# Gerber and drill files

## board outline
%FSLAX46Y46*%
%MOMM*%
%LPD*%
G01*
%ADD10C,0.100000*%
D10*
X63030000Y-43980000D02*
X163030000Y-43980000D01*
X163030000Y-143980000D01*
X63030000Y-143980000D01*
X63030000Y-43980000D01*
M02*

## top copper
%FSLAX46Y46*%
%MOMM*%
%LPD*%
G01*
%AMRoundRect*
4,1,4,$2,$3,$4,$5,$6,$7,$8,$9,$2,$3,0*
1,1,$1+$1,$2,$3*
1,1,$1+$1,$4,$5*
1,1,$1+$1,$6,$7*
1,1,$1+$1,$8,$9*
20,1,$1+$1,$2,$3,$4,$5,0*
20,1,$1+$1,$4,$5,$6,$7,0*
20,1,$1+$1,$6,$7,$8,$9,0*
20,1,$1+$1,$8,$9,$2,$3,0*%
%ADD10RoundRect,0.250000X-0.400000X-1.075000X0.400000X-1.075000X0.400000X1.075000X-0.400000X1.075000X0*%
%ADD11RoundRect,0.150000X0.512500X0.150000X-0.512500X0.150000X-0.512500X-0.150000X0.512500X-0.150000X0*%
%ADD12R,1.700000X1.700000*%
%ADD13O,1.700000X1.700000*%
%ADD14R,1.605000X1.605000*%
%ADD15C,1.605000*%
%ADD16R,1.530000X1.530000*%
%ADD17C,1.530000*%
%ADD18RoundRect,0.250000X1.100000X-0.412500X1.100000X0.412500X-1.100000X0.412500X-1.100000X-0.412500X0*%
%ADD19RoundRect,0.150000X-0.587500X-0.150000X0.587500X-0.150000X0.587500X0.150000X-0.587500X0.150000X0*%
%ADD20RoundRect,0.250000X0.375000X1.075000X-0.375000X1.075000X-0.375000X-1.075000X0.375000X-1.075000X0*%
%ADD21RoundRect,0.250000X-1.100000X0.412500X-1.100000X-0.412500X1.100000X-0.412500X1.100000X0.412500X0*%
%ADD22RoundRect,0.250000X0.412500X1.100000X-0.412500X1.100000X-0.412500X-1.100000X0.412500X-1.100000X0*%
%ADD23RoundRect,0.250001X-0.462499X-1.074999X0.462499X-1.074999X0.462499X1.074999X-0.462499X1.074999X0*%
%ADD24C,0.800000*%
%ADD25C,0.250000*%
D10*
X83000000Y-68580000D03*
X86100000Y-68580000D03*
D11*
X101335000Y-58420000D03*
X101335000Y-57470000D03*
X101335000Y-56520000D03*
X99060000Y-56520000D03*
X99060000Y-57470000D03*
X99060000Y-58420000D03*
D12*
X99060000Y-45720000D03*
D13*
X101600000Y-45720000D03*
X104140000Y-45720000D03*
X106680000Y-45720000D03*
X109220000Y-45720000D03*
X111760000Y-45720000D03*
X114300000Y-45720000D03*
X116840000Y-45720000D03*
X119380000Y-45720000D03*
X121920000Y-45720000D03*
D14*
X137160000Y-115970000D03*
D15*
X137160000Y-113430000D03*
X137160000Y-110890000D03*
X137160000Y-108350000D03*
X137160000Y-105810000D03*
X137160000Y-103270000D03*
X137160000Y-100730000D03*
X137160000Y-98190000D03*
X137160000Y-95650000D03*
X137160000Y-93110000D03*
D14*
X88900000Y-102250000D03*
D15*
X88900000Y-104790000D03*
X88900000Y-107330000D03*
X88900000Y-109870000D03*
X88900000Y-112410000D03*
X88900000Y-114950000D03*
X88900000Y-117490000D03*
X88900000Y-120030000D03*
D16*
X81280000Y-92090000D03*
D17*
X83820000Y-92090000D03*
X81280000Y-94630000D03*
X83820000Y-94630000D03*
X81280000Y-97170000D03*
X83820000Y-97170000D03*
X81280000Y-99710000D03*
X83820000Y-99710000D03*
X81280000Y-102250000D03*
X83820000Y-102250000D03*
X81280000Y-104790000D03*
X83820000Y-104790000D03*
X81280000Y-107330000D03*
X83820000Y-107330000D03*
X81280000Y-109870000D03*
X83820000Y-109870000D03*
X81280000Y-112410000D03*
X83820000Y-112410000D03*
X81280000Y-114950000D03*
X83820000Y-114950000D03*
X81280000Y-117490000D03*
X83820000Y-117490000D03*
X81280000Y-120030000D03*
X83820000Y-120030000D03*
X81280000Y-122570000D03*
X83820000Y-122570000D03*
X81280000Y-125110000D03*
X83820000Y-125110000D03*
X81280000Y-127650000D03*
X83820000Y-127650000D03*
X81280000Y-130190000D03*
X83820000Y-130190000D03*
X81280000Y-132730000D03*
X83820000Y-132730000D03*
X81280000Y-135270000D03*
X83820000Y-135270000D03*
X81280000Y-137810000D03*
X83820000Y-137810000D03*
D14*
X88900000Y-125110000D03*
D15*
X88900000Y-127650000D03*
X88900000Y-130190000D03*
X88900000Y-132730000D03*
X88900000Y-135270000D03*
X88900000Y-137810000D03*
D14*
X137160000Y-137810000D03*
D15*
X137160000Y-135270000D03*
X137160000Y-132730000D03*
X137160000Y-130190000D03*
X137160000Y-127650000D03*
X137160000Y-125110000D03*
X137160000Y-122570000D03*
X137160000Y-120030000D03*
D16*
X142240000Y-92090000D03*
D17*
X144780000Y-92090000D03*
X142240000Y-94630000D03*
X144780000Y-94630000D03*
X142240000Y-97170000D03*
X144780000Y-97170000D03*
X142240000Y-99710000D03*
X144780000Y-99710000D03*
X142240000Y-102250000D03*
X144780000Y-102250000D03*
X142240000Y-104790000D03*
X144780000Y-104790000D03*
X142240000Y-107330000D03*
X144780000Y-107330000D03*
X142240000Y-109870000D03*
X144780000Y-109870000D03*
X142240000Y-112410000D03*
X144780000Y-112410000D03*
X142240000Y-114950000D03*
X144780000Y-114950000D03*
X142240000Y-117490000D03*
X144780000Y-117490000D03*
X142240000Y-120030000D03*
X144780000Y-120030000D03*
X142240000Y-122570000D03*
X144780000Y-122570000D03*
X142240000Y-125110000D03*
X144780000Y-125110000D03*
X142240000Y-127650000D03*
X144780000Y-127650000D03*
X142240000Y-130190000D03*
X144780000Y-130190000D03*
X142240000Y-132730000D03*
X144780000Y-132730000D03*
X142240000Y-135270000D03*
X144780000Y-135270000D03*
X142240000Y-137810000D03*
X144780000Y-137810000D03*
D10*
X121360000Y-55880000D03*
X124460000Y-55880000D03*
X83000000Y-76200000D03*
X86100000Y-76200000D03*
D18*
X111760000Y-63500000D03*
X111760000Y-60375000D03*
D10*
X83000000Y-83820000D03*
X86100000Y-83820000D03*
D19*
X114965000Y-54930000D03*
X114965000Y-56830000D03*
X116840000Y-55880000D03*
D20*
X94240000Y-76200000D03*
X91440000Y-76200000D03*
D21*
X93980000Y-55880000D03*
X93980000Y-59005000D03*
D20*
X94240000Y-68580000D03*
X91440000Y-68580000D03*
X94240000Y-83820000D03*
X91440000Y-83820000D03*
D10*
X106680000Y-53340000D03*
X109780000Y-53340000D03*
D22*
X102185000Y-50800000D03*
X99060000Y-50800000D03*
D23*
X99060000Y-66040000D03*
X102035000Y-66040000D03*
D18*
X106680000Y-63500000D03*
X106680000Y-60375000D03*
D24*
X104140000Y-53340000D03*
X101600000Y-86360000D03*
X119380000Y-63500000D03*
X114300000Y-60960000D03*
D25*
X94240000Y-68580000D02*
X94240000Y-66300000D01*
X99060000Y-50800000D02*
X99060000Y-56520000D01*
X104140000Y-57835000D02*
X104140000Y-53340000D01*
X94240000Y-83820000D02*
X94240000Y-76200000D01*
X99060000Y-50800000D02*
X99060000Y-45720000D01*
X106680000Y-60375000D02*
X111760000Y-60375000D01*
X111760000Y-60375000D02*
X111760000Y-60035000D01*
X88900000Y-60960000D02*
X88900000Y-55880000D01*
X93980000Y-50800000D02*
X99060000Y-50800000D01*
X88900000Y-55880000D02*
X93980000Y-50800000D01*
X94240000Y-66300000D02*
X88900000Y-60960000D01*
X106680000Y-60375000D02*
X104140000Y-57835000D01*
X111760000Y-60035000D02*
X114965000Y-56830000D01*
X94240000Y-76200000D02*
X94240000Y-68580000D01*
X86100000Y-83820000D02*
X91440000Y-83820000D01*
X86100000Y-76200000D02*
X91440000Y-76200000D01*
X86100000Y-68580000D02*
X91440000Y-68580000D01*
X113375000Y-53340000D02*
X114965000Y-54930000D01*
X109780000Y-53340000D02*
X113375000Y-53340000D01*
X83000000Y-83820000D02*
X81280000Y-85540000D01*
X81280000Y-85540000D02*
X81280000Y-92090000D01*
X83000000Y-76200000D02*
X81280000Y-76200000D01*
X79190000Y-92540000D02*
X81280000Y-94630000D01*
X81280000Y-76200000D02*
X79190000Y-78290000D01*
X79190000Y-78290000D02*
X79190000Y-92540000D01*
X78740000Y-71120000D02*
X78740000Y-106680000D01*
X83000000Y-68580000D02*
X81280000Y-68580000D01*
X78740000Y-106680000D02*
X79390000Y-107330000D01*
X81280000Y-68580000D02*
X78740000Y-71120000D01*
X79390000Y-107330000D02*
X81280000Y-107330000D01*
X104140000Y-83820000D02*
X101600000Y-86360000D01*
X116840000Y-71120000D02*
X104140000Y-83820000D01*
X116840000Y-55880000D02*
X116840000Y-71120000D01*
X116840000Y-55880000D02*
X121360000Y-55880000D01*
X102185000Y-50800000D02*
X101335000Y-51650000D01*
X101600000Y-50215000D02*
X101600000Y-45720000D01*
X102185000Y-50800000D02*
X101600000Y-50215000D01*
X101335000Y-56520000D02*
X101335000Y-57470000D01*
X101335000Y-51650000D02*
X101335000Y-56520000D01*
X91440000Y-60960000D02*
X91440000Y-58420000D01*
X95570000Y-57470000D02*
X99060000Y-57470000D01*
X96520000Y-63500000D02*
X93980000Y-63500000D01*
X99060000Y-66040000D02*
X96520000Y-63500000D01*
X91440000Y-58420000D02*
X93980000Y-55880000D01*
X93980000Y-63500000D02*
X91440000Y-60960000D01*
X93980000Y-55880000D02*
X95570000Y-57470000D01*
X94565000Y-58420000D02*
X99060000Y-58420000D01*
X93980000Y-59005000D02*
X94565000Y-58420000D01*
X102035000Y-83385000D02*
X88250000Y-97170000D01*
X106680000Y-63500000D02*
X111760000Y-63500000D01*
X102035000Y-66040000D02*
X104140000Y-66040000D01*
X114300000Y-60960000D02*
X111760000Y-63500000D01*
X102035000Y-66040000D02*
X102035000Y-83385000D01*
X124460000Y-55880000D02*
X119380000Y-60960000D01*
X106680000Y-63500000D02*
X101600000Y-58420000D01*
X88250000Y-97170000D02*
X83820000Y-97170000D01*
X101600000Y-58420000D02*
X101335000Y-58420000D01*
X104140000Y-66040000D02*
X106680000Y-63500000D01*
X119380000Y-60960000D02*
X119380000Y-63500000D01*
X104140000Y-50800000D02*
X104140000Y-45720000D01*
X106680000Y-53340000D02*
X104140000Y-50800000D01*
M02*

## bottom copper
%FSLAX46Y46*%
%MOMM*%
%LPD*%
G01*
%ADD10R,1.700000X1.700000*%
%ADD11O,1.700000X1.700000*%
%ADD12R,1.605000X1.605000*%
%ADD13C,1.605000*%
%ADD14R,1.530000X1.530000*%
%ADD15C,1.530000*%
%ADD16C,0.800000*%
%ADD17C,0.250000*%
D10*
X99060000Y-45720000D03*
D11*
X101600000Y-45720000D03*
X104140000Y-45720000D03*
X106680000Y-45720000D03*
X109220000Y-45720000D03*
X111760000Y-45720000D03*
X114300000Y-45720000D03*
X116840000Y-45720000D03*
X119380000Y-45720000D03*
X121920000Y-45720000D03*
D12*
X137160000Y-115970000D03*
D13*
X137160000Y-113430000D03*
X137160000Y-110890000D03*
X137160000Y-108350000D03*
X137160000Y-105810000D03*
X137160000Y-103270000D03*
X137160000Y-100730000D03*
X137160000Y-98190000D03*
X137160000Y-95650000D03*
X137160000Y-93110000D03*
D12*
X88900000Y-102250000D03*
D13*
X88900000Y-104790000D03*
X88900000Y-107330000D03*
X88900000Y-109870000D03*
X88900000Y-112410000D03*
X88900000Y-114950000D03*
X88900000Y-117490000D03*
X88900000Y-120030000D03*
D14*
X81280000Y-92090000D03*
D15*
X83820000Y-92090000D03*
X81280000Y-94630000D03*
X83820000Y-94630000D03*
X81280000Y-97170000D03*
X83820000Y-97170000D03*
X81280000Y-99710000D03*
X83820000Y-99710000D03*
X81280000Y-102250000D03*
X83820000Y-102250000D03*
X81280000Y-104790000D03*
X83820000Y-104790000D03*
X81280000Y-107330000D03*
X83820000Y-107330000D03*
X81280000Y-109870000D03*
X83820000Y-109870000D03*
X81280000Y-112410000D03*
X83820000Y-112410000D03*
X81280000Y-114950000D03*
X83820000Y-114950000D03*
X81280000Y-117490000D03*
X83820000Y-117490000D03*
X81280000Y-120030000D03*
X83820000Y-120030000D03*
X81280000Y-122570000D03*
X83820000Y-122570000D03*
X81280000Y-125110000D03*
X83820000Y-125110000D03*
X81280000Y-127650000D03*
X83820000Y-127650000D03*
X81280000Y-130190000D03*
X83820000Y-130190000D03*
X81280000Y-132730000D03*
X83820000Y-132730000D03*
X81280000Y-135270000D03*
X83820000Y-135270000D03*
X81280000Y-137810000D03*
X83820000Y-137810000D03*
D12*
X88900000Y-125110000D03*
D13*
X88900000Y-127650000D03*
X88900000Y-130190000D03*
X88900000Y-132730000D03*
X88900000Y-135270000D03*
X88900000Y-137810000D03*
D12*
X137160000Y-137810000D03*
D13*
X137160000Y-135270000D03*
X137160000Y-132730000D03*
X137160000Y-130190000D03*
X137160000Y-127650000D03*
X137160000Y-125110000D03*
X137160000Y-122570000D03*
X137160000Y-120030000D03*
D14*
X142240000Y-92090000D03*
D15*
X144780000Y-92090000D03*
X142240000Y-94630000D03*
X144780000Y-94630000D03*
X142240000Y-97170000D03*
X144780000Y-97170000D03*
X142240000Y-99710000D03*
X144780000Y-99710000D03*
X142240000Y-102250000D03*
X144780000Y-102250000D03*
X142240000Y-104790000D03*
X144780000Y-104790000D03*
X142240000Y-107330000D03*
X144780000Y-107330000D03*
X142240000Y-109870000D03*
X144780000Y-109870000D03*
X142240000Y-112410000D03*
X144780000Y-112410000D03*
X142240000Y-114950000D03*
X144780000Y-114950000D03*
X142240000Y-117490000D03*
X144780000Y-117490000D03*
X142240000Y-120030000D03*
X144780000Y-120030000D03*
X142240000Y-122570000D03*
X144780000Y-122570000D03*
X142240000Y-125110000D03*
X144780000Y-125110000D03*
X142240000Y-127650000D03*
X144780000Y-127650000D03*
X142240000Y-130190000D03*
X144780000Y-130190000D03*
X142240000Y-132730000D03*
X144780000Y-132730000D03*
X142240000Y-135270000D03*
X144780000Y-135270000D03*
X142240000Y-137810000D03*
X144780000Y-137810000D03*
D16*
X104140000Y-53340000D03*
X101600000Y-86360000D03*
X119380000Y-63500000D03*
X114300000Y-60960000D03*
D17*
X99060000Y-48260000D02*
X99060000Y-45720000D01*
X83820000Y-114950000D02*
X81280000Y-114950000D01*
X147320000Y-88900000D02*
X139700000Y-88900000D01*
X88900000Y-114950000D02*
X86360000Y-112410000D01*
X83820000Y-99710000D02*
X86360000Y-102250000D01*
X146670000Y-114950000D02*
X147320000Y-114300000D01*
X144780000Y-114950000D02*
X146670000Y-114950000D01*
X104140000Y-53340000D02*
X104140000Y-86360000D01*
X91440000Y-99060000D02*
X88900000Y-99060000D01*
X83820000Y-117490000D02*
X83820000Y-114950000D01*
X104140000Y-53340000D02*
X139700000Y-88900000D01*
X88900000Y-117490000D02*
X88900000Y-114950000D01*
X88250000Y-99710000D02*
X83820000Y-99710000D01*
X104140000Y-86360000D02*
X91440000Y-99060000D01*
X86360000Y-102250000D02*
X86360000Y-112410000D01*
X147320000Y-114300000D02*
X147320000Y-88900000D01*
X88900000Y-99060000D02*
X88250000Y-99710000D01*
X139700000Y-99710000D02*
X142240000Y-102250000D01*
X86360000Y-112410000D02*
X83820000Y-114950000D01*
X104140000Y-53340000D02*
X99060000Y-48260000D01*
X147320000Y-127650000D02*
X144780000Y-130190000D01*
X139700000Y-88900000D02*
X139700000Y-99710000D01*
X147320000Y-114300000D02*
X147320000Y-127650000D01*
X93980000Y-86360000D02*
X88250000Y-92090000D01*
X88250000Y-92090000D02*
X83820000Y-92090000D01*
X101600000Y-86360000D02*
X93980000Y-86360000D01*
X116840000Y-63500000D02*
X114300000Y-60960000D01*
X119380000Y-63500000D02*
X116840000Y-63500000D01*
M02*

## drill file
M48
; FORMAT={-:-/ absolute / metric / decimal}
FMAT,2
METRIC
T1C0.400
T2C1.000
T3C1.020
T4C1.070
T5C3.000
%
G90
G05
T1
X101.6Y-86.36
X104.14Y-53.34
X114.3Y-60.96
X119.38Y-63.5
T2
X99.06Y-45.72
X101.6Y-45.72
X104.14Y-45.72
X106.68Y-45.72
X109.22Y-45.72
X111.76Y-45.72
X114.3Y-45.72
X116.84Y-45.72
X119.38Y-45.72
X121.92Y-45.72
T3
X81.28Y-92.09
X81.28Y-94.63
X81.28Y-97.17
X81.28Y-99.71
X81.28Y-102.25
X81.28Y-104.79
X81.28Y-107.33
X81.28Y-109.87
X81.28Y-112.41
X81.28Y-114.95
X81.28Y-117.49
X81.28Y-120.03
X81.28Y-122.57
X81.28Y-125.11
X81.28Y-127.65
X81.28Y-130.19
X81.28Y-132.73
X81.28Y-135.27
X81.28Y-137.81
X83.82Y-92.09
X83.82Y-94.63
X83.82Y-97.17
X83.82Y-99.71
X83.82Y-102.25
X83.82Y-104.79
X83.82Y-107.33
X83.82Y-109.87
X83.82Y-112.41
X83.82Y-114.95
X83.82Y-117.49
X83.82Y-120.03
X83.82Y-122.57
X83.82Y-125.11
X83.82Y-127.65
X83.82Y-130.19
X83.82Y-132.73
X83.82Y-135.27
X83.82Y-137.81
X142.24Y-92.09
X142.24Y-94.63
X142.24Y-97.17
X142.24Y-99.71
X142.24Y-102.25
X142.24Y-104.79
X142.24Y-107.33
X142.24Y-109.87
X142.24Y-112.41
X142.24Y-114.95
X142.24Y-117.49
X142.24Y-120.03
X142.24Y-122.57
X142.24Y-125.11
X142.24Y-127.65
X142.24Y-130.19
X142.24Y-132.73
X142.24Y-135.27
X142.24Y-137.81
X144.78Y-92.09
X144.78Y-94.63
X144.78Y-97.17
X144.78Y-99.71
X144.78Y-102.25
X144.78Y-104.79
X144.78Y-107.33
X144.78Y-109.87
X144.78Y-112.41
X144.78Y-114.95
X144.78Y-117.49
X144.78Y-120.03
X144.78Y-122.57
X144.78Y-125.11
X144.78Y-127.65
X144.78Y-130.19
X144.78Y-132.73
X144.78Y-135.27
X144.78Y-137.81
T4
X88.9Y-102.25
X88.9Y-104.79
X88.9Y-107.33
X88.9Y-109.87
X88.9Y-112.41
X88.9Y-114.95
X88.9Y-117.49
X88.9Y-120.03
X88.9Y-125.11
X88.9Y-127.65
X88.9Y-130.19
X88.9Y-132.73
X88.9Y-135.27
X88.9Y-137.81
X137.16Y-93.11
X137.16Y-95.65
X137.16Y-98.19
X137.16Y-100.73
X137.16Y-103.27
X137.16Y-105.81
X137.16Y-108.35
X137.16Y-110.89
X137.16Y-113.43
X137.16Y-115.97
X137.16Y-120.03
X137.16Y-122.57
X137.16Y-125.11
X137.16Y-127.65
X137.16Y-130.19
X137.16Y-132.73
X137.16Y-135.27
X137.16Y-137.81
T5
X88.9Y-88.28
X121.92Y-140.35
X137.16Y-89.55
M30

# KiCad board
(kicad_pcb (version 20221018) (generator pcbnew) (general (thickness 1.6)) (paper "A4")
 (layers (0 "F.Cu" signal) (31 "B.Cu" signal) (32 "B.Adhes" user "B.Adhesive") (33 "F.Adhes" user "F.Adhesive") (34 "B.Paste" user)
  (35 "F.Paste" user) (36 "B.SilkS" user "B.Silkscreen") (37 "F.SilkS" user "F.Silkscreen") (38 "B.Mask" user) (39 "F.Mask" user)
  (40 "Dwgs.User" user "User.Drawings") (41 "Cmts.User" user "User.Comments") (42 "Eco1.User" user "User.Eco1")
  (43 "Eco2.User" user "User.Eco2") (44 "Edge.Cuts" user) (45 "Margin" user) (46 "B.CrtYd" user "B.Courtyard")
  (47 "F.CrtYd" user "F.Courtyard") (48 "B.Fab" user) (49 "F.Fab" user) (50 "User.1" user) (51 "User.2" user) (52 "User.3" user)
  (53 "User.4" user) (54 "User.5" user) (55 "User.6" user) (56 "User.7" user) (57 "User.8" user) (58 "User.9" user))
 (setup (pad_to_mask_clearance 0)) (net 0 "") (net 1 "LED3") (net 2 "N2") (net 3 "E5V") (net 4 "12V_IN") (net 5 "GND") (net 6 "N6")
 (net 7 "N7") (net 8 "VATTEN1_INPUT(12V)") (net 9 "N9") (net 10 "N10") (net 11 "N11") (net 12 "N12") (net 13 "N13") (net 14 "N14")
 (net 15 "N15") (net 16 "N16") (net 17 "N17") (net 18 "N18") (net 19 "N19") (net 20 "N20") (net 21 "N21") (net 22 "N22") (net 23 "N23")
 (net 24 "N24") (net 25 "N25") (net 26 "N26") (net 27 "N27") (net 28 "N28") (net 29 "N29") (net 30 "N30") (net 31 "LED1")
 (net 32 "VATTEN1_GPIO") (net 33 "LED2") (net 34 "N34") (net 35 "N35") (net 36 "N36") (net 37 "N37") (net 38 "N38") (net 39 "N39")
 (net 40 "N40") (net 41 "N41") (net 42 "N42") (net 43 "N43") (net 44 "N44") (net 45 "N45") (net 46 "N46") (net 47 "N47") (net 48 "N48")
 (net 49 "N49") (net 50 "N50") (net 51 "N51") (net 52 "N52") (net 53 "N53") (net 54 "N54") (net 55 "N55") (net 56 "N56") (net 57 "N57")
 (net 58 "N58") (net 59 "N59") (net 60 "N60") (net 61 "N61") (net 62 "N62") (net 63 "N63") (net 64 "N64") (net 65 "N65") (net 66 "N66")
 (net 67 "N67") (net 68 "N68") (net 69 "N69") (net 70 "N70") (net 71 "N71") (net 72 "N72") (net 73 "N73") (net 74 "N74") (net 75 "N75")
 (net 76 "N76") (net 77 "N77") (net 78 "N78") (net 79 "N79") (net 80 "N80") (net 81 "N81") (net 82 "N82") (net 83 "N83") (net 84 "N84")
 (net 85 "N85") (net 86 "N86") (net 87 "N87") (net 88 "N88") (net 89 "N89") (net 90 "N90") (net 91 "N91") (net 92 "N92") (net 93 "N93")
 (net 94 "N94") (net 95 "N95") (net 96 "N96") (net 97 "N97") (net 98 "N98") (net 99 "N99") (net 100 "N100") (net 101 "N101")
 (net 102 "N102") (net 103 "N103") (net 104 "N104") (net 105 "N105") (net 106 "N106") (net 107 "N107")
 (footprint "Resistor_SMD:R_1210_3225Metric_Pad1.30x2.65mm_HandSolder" (layer "F.Cu") (at 84.55 68.58)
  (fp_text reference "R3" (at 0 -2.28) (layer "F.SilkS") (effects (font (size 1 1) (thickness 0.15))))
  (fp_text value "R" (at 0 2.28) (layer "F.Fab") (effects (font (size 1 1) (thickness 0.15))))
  (pad "1" smd roundrect (at -1.55 0) (size 1.3 2.65) (layers "F.Cu" "F.Paste" "F.Mask") (roundrect_rratio 0.192308) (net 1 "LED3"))
  (pad "2" smd roundrect (at 1.55 0) (size 1.3 2.65) (layers "F.Cu" "F.Paste" "F.Mask") (roundrect_rratio 0.192308) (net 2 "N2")))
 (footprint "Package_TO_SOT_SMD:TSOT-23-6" (layer "F.Cu") (at 100.1975 57.47 180)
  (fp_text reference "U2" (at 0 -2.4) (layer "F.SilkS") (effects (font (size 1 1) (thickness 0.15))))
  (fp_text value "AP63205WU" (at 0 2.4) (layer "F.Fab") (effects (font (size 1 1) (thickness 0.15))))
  (pad "1" smd roundrect (at -1.1375 -0.95 180) (size 1.325 0.6) (layers "F.Cu" "F.Paste" "F.Mask") (roundrect_rratio 0.25) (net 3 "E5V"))
  (pad "2" smd roundrect (at -1.1375 0 180) (size 1.325 0.6) (layers "F.Cu" "F.Paste" "F.Mask") (roundrect_rratio 0.25) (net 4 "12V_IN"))
  (pad "3" smd roundrect (at -1.1375 0.95 180) (size 1.325 0.6) (layers "F.Cu" "F.Paste" "F.Mask") (roundrect_rratio 0.25) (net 4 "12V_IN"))
  (pad "4" smd roundrect (at 1.1375 0.95 180) (size 1.325 0.6) (layers "F.Cu" "F.Paste" "F.Mask") (roundrect_rratio 0.25) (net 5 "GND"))
  (pad "5" smd roundrect (at 1.1375 0 180) (size 1.325 0.6) (layers "F.Cu" "F.Paste" "F.Mask") (roundrect_rratio 0.25) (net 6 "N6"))
  (pad "6" smd roundrect (at 1.1375 -0.95 180) (size 1.325 0.6) (layers "F.Cu" "F.Paste" "F.Mask") (roundrect_rratio 0.25) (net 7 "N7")))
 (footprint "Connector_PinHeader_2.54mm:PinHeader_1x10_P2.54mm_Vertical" (layer "F.Cu") (at 99.06 45.72 90)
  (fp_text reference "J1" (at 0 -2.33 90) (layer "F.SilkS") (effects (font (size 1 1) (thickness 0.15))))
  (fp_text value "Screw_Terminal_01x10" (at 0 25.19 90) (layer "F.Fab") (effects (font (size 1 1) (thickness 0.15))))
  (pad "1" thru_hole rect (at 0 0 90) (size 1.7 1.7) (drill 1) (layers "*.Cu" "*.Mask") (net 5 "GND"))
  (pad "2" thru_hole oval (at 0 2.54 90) (size 1.7 1.7) (drill 1) (layers "*.Cu" "*.Mask") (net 4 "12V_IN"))
  (pad "3" thru_hole oval (at 0 5.08 90) (size 1.7 1.7) (drill 1) (layers "*.Cu" "*.Mask") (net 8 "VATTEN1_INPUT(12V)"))
  (pad "4" thru_hole oval (at 0 7.62 90) (size 1.7 1.7) (drill 1) (layers "*.Cu" "*.Mask") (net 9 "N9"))
  (pad "5" thru_hole oval (at 0 10.16 90) (size 1.7 1.7) (drill 1) (layers "*.Cu" "*.Mask") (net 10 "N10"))
  (pad "6" thru_hole oval (at 0 12.7 90) (size 1.7 1.7) (drill 1) (layers "*.Cu" "*.Mask") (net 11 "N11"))
  (pad "7" thru_hole oval (at 0 15.24 90) (size 1.7 1.7) (drill 1) (layers "*.Cu" "*.Mask") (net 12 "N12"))
  (pad "8" thru_hole oval (at 0 17.78 90) (size 1.7 1.7) (drill 1) (layers "*.Cu" "*.Mask") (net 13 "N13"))
  (pad "9" thru_hole oval (at 0 20.32 90) (size 1.7 1.7) (drill 1) (layers "*.Cu" "*.Mask") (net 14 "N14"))
  (pad "10" thru_hole oval (at 0 22.86 90) (size 1.7 1.7) (drill 1) (layers "*.Cu" "*.Mask") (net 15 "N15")))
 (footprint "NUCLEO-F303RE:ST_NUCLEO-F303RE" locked (layer "F.Cu") (at 113.03 101.6)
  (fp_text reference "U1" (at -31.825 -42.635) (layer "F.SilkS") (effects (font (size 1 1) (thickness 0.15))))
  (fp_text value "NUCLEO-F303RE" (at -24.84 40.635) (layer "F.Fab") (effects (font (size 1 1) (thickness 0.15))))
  (pad "" np_thru_hole circle locked (at -24.13 -13.32) (size 3 3) (drill 3) (layers "*.Cu" "*.Mask"))
  (pad "" np_thru_hole circle locked (at 8.89 38.75) (size 3 3) (drill 3) (layers "*.Cu" "*.Mask"))
  (pad "" np_thru_hole circle locked (at 24.13 -12.05) (size 3 3) (drill 3) (layers "*.Cu" "*.Mask"))
  (pad "CN5_1" thru_hole rect locked (at 24.13 14.37) (size 1.605 1.605) (drill 1.07) (layers "*.Cu" "*.Mask") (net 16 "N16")
   (solder_mask_margin 0.102))
  (pad "CN5_2" thru_hole circle locked (at 24.13 11.83) (size 1.605 1.605) (drill 1.07) (layers "*.Cu" "*.Mask") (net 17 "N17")
   (solder_mask_margin 0.102))
  (pad "CN5_3" thru_hole circle locked (at 24.13 9.29) (size 1.605 1.605) (drill 1.07) (layers "*.Cu" "*.Mask") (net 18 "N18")
   (solder_mask_margin 0.102))
  (pad "CN5_4" thru_hole circle locked (at 24.13 6.75) (size 1.605 1.605) (drill 1.07) (layers "*.Cu" "*.Mask") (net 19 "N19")
   (solder_mask_margin 0.102))
  (pad "CN5_5" thru_hole circle locked (at 24.13 4.21) (size 1.605 1.605) (drill 1.07) (layers "*.Cu" "*.Mask") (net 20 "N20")
   (solder_mask_margin 0.102))
  (pad "CN5_6" thru_hole circle locked (at 24.13 1.67) (size 1.605 1.605) (drill 1.07) (layers "*.Cu" "*.Mask") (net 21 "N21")
   (solder_mask_margin 0.102))
  (pad "CN5_7" thru_hole circle locked (at 24.13 -0.87) (size 1.605 1.605) (drill 1.07) (layers "*.Cu" "*.Mask") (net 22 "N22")
   (solder_mask_margin 0.102))
  (pad "CN5_8" thru_hole circle locked (at 24.13 -3.41) (size 1.605 1.605) (drill 1.07) (layers "*.Cu" "*.Mask") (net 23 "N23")
   (solder_mask_margin 0.102))
  (pad "CN5_9" thru_hole circle locked (at 24.13 -5.95) (size 1.605 1.605) (drill 1.07) (layers "*.Cu" "*.Mask") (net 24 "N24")
   (solder_mask_margin 0.102))
  (pad "CN5_10" thru_hole circle locked (at 24.13 -8.49) (size 1.605 1.605) (drill 1.07) (layers "*.Cu" "*.Mask") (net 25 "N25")
   (solder_mask_margin 0.102))
  (pad "CN6_1" thru_hole rect locked (at -24.13 0.65) (size 1.605 1.605) (drill 1.07) (layers "*.Cu" "*.Mask") (solder_mask_margin 0.102))
  (pad "CN6_2" thru_hole circle locked (at -24.13 3.19) (size 1.605 1.605) (drill 1.07) (layers "*.Cu" "*.Mask") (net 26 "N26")
   (solder_mask_margin 0.102))
  (pad "CN6_3" thru_hole circle locked (at -24.13 5.73) (size 1.605 1.605) (drill 1.07) (layers "*.Cu" "*.Mask") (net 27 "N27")
   (solder_mask_margin 0.102))
  (pad "CN6_4" thru_hole circle locked (at -24.13 8.27) (size 1.605 1.605) (drill 1.07) (layers "*.Cu" "*.Mask") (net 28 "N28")
   (solder_mask_margin 0.102))
  (pad "CN6_5" thru_hole circle locked (at -24.13 10.81) (size 1.605 1.605) (drill 1.07) (layers "*.Cu" "*.Mask") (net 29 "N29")
   (solder_mask_margin 0.102))
  (pad "CN6_6" thru_hole circle locked (at -24.13 13.35) (size 1.605 1.605) (drill 1.07) (layers "*.Cu" "*.Mask") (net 5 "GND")
   (solder_mask_margin 0.102))
  (pad "CN6_7" thru_hole circle locked (at -24.13 15.89) (size 1.605 1.605) (drill 1.07) (layers "*.Cu" "*.Mask") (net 5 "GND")
   (solder_mask_margin 0.102))
  (pad "CN6_8" thru_hole circle locked (at -24.13 18.43) (size 1.605 1.605) (drill 1.07) (layers "*.Cu" "*.Mask") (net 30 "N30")
   (solder_mask_margin 0.102))
  (pad "CN7_1" thru_hole rect locked (at -31.75 -9.51) (size 1.53 1.53) (drill 1.02) (layers "*.Cu" "*.Mask") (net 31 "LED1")
   (solder_mask_margin 0.102))
  (pad "CN7_2" thru_hole circle locked (at -29.21 -9.51) (size 1.53 1.53) (drill 1.02) (layers "*.Cu" "*.Mask") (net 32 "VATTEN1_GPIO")
   (solder_mask_margin 0.102))
  (pad "CN7_3" thru_hole circle locked (at -31.75 -6.97) (size 1.53 1.53) (drill 1.02) (layers "*.Cu" "*.Mask") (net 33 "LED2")
   (solder_mask_margin 0.102))
  (pad "CN7_4" thru_hole circle locked (at -29.21 -6.97) (size 1.53 1.53) (drill 1.02) (layers "*.Cu" "*.Mask") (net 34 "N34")
   (solder_mask_margin 0.102))
  (pad "CN7_5" thru_hole circle locked (at -31.75 -4.43) (size 1.53 1.53) (drill 1.02) (layers "*.Cu" "*.Mask") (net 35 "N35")
   (solder_mask_margin 0.102))
  (pad "CN7_6" thru_hole circle locked (at -29.21 -4.43) (size 1.53 1.53) (drill 1.02) (layers "*.Cu" "*.Mask") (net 3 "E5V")
   (solder_mask_margin 0.102))
  (pad "CN7_7" thru_hole circle locked (at -31.75 -1.89) (size 1.53 1.53) (drill 1.02) (layers "*.Cu" "*.Mask") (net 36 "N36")
   (solder_mask_margin 0.102))
  (pad "CN7_8" thru_hole circle locked (at -29.21 -1.89) (size 1.53 1.53) (drill 1.02) (layers "*.Cu" "*.Mask") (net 5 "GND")
   (solder_mask_margin 0.102))
  (pad "CN7_9" thru_hole circle locked (at -31.75 0.65) (size 1.53 1.53) (drill 1.02) (layers "*.Cu" "*.Mask") (solder_mask_margin 0.102))
  (pad "CN7_10" thru_hole circle locked (at -29.21 0.65) (size 1.53 1.53) (drill 1.02) (layers "*.Cu" "*.Mask") (solder_mask_margin 0.102))
  (pad "CN7_11" thru_hole circle locked (at -31.75 3.19) (size 1.53 1.53) (drill 1.02) (layers "*.Cu" "*.Mask") (solder_mask_margin 0.102))
  (pad "CN7_12" thru_hole circle locked (at -29.21 3.19) (size 1.53 1.53) (drill 1.02) (layers "*.Cu" "*.Mask") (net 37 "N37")
   (solder_mask_margin 0.102))
  (pad "CN7_13" thru_hole circle locked (at -31.75 5.73) (size 1.53 1.53) (drill 1.02) (layers "*.Cu" "*.Mask") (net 1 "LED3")
   (solder_mask_margin 0.102))
  (pad "CN7_14" thru_hole circle locked (at -29.21 5.73) (size 1.53 1.53) (drill 1.02) (layers "*.Cu" "*.Mask") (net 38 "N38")
   (solder_mask_margin 0.102))
  (pad "CN7_15" thru_hole circle locked (at -31.75 8.27) (size 1.53 1.53) (drill 1.02) (layers "*.Cu" "*.Mask") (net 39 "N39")
   (solder_mask_margin 0.102))
  (pad "CN7_16" thru_hole circle locked (at -29.21 8.27) (size 1.53 1.53) (drill 1.02) (layers "*.Cu" "*.Mask") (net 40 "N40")
   (solder_mask_margin 0.102))
  (pad "CN7_17" thru_hole circle locked (at -31.75 10.81) (size 1.53 1.53) (drill 1.02) (layers "*.Cu" "*.Mask") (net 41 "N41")
   (solder_mask_margin 0.102))
  (pad "CN7_18" thru_hole circle locked (at -29.21 10.81) (size 1.53 1.53) (drill 1.02) (layers "*.Cu" "*.Mask") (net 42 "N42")
   (solder_mask_margin 0.102))
  (pad "CN7_19" thru_hole circle locked (at -31.75 13.35) (size 1.53 1.53) (drill 1.02) (layers "*.Cu" "*.Mask") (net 5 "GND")
   (solder_mask_margin 0.102))
  (pad "CN7_20" thru_hole circle locked (at -29.21 13.35) (size 1.53 1.53) (drill 1.02) (layers "*.Cu" "*.Mask") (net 5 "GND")
   (solder_mask_margin 0.102))
  (pad "CN7_21" thru_hole circle locked (at -31.75 15.89) (size 1.53 1.53) (drill 1.02) (layers "*.Cu" "*.Mask") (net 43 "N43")
   (solder_mask_margin 0.102))
  (pad "CN7_22" thru_hole circle locked (at -29.21 15.89) (size 1.53 1.53) (drill 1.02) (layers "*.Cu" "*.Mask") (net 5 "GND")
   (solder_mask_margin 0.102))
  (pad "CN7_23" thru_hole circle locked (at -31.75 18.43) (size 1.53 1.53) (drill 1.02) (layers "*.Cu" "*.Mask") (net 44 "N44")
   (solder_mask_margin 0.102))
  (pad "CN7_24" thru_hole circle locked (at -29.21 18.43) (size 1.53 1.53) (drill 1.02) (layers "*.Cu" "*.Mask") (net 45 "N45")
   (solder_mask_margin 0.102))
  (pad "CN7_25" thru_hole circle locked (at -31.75 20.97) (size 1.53 1.53) (drill 1.02) (layers "*.Cu" "*.Mask") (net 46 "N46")
   (solder_mask_margin 0.102))
  (pad "CN7_26" thru_hole circle locked (at -29.21 20.97) (size 1.53 1.53) (drill 1.02) (layers "*.Cu" "*.Mask") (solder_mask_margin 0.102))
  (pad "CN7_27" thru_hole circle locked (at -31.75 23.51) (size 1.53 1.53) (drill 1.02) (layers "*.Cu" "*.Mask") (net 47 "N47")
   (solder_mask_margin 0.102))
  (pad "CN7_28" thru_hole circle locked (at -29.21 23.51) (size 1.53 1.53) (drill 1.02) (layers "*.Cu" "*.Mask") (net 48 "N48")
   (solder_mask_margin 0.102))
  (pad "CN7_29" thru_hole circle locked (at -31.75 26.05) (size 1.53 1.53) (drill 1.02) (layers "*.Cu" "*.Mask") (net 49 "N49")
   (solder_mask_margin 0.102))
  (pad "CN7_30" thru_hole circle locked (at -29.21 26.05) (size 1.53 1.53) (drill 1.02) (layers "*.Cu" "*.Mask") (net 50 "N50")
   (solder_mask_margin 0.102))
  (pad "CN7_31" thru_hole circle locked (at -31.75 28.59) (size 1.53 1.53) (drill 1.02) (layers "*.Cu" "*.Mask") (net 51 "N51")
   (solder_mask_margin 0.102))
  (pad "CN7_32" thru_hole circle locked (at -29.21 28.59) (size 1.53 1.53) (drill 1.02) (layers "*.Cu" "*.Mask") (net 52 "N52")
   (solder_mask_margin 0.102))
  (pad "CN7_33" thru_hole circle locked (at -31.75 31.13) (size 1.53 1.53) (drill 1.02) (layers "*.Cu" "*.Mask") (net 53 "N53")
   (solder_mask_margin 0.102))
  (pad "CN7_34" thru_hole circle locked (at -29.21 31.13) (size 1.53 1.53) (drill 1.02) (layers "*.Cu" "*.Mask") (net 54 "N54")
   (solder_mask_margin 0.102))
  (pad "CN7_35" thru_hole circle locked (at -31.75 33.67) (size 1.53 1.53) (drill 1.02) (layers "*.Cu" "*.Mask") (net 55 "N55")
   (solder_mask_margin 0.102))
  (pad "CN7_36" thru_hole circle locked (at -29.21 33.67) (size 1.53 1.53) (drill 1.02) (layers "*.Cu" "*.Mask") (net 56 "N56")
   (solder_mask_margin 0.102))
  (pad "CN7_37" thru_hole circle locked (at -31.75 36.21) (size 1.53 1.53) (drill 1.02) (layers "*.Cu" "*.Mask") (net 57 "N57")
   (solder_mask_margin 0.102))
  (pad "CN7_38" thru_hole circle locked (at -29.21 36.21) (size 1.53 1.53) (drill 1.02) (layers "*.Cu" "*.Mask") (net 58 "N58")
   (solder_mask_margin 0.102))
  (pad "CN8_1" thru_hole rect locked (at -24.13 23.51) (size 1.605 1.605) (drill 1.07) (layers "*.Cu" "*.Mask") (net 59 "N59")
   (solder_mask_margin 0.102))
  (pad "CN8_2" thru_hole circle locked (at -24.13 26.05) (size 1.605 1.605) (drill 1.07) (layers "*.Cu" "*.Mask") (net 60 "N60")
   (solder_mask_margin 0.102))
  (pad "CN8_3" thru_hole circle locked (at -24.13 28.59) (size 1.605 1.605) (drill 1.07) (layers "*.Cu" "*.Mask") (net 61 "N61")
   (solder_mask_margin 0.102))
  (pad "CN8_4" thru_hole circle locked (at -24.13 31.13) (size 1.605 1.605) (drill 1.07) (layers "*.Cu" "*.Mask") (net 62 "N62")
   (solder_mask_margin 0.102))
  (pad "CN8_5" thru_hole circle locked (at -24.13 33.67) (size 1.605 1.605) (drill 1.07) (layers "*.Cu" "*.Mask") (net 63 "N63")
   (solder_mask_margin 0.102))
  (pad "CN8_6" thru_hole circle locked (at -24.13 36.21) (size 1.605 1.605) (drill 1.07) (layers "*.Cu" "*.Mask") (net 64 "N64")
   (solder_mask_margin 0.102))
  (pad "CN9_1" thru_hole rect locked (at 24.13 36.21) (size 1.605 1.605) (drill 1.07) (layers "*.Cu" "*.Mask") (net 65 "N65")
   (solder_mask_margin 0.102))
  (pad "CN9_2" thru_hole circle locked (at 24.13 33.67) (size 1.605 1.605) (drill 1.07) (layers "*.Cu" "*.Mask") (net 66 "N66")
   (solder_mask_margin 0.102))
  (pad "CN9_3" thru_hole circle locked (at 24.13 31.13) (size 1.605 1.605) (drill 1.07) (layers "*.Cu" "*.Mask") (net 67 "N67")
   (solder_mask_margin 0.102))
  (pad "CN9_4" thru_hole circle locked (at 24.13 28.59) (size 1.605 1.605) (drill 1.07) (layers "*.Cu" "*.Mask") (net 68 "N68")
   (solder_mask_margin 0.102))
  (pad "CN9_5" thru_hole circle locked (at 24.13 26.05) (size 1.605 1.605) (drill 1.07) (layers "*.Cu" "*.Mask") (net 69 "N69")
   (solder_mask_margin 0.102))
  (pad "CN9_6" thru_hole circle locked (at 24.13 23.51) (size 1.605 1.605) (drill 1.07) (layers "*.Cu" "*.Mask") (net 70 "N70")
   (solder_mask_margin 0.102))
  (pad "CN9_7" thru_hole circle locked (at 24.13 20.97) (size 1.605 1.605) (drill 1.07) (layers "*.Cu" "*.Mask") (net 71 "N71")
   (solder_mask_margin 0.102))
  (pad "CN9_8" thru_hole circle locked (at 24.13 18.43) (size 1.605 1.605) (drill 1.07) (layers "*.Cu" "*.Mask") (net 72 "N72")
   (solder_mask_margin 0.102))
  (pad "CN10_1" thru_hole rect locked (at 29.21 -9.51) (size 1.53 1.53) (drill 1.02) (layers "*.Cu" "*.Mask") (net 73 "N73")
   (solder_mask_margin 0.102))
  (pad "CN10_2" thru_hole circle locked (at 31.75 -9.51) (size 1.53 1.53) (drill 1.02) (layers "*.Cu" "*.Mask") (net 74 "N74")
   (solder_mask_margin 0.102))
  (pad "CN10_3" thru_hole circle locked (at 29.21 -6.97) (size 1.53 1.53) (drill 1.02) (layers "*.Cu" "*.Mask") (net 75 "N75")
   (solder_mask_margin 0.102))
  (pad "CN10_4" thru_hole circle locked (at 31.75 -6.97) (size 1.53 1.53) (drill 1.02) (layers "*.Cu" "*.Mask") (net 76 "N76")
   (solder_mask_margin 0.102))
  (pad "CN10_5" thru_hole circle locked (at 29.21 -4.43) (size 1.53 1.53) (drill 1.02) (layers "*.Cu" "*.Mask") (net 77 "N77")
   (solder_mask_margin 0.102))
  (pad "CN10_6" thru_hole circle locked (at 31.75 -4.43) (size 1.53 1.53) (drill 1.02) (layers "*.Cu" "*.Mask") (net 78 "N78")
   (solder_mask_margin 0.102))
  (pad "CN10_7" thru_hole circle locked (at 29.21 -1.89) (size 1.53 1.53) (drill 1.02) (layers "*.Cu" "*.Mask") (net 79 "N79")
   (solder_mask_margin 0.102))
  (pad "CN10_8" thru_hole circle locked (at 31.75 -1.89) (size 1.53 1.53) (drill 1.02) (layers "*.Cu" "*.Mask") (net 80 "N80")
   (solder_mask_margin 0.102))
  (pad "CN10_9" thru_hole circle locked (at 29.21 0.65) (size 1.53 1.53) (drill 1.02) (layers "*.Cu" "*.Mask") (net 5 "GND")
   (solder_mask_margin 0.102))
  (pad "CN10_10" thru_hole circle locked (at 31.75 0.65) (size 1.53 1.53) (drill 1.02) (layers "*.Cu" "*.Mask") (solder_mask_margin 0.102))
  (pad "CN10_11" thru_hole circle locked (at 29.21 3.19) (size 1.53 1.53) (drill 1.02) (layers "*.Cu" "*.Mask") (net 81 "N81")
   (solder_mask_margin 0.102))
  (pad "CN10_12" thru_hole circle locked (at 31.75 3.19) (size 1.53 1.53) (drill 1.02) (layers "*.Cu" "*.Mask") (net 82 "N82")
   (solder_mask_margin 0.102))
  (pad "CN10_13" thru_hole circle locked (at 29.21 5.73) (size 1.53 1.53) (drill 1.02) (layers "*.Cu" "*.Mask") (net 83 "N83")
   (solder_mask_margin 0.102))
  (pad "CN10_14" thru_hole circle locked (at 31.75 5.73) (size 1.53 1.53) (drill 1.02) (layers "*.Cu" "*.Mask") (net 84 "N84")
   (solder_mask_margin 0.102))
  (pad "CN10_15" thru_hole circle locked (at 29.21 8.27) (size 1.53 1.53) (drill 1.02) (layers "*.Cu" "*.Mask") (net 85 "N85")
   (solder_mask_margin 0.102))
  (pad "CN10_16" thru_hole circle locked (at 31.75 8.27) (size 1.53 1.53) (drill 1.02) (layers "*.Cu" "*.Mask") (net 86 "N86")
   (solder_mask_margin 0.102))
  (pad "CN10_17" thru_hole circle locked (at 29.21 10.81) (size 1.53 1.53) (drill 1.02) (layers "*.Cu" "*.Mask") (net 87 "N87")
   (solder_mask_margin 0.102))
  (pad "CN10_18" thru_hole circle locked (at 31.75 10.81) (size 1.53 1.53) (drill 1.02) (layers "*.Cu" "*.Mask") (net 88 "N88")
   (solder_mask_margin 0.102))
  (pad "CN10_19" thru_hole circle locked (at 29.21 13.35) (size 1.53 1.53) (drill 1.02) (layers "*.Cu" "*.Mask") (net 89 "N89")
   (solder_mask_margin 0.102))
  (pad "CN10_20" thru_hole circle locked (at 31.75 13.35) (size 1.53 1.53) (drill 1.02) (layers "*.Cu" "*.Mask") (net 5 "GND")
   (solder_mask_margin 0.102))
  (pad "CN10_21" thru_hole circle locked (at 29.21 15.89) (size 1.53 1.53) (drill 1.02) (layers "*.Cu" "*.Mask") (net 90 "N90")
   (solder_mask_margin 0.102))
  (pad "CN10_22" thru_hole circle locked (at 31.75 15.89) (size 1.53 1.53) (drill 1.02) (layers "*.Cu" "*.Mask") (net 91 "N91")
   (solder_mask_margin 0.102))
  (pad "CN10_23" thru_hole circle locked (at 29.21 18.43) (size 1.53 1.53) (drill 1.02) (layers "*.Cu" "*.Mask") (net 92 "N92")
   (solder_mask_margin 0.102))
  (pad "CN10_24" thru_hole circle locked (at 31.75 18.43) (size 1.53 1.53) (drill 1.02) (layers "*.Cu" "*.Mask") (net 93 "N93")
   (solder_mask_margin 0.102))
  (pad "CN10_25" thru_hole circle locked (at 29.21 20.97) (size 1.53 1.53) (drill 1.02) (layers "*.Cu" "*.Mask") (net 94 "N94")
   (solder_mask_margin 0.102))
  (pad "CN10_26" thru_hole circle locked (at 31.75 20.97) (size 1.53 1.53) (drill 1.02) (layers "*.Cu" "*.Mask") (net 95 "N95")
   (solder_mask_margin 0.102))
  (pad "CN10_27" thru_hole circle locked (at 29.21 23.51) (size 1.53 1.53) (drill 1.02) (layers "*.Cu" "*.Mask") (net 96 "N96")
   (solder_mask_margin 0.102))
  (pad "CN10_28" thru_hole circle locked (at 31.75 23.51) (size 1.53 1.53) (drill 1.02) (layers "*.Cu" "*.Mask") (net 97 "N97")
   (solder_mask_margin 0.102))
  (pad "CN10_29" thru_hole circle locked (at 29.21 26.05) (size 1.53 1.53) (drill 1.02) (layers "*.Cu" "*.Mask") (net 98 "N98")
   (solder_mask_margin 0.102))
  (pad "CN10_30" thru_hole circle locked (at 31.75 26.05) (size 1.53 1.53) (drill 1.02) (layers "*.Cu" "*.Mask") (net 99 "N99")
   (solder_mask_margin 0.102))
  (pad "CN10_31" thru_hole circle locked (at 29.21 28.59) (size 1.53 1.53) (drill 1.02) (layers "*.Cu" "*.Mask") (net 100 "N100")
   (solder_mask_margin 0.102))
  (pad "CN10_32" thru_hole circle locked (at 31.75 28.59) (size 1.53 1.53) (drill 1.02) (layers "*.Cu" "*.Mask") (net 5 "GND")
   (solder_mask_margin 0.102))
  (pad "CN10_33" thru_hole circle locked (at 29.21 31.13) (size 1.53 1.53) (drill 1.02) (layers "*.Cu" "*.Mask") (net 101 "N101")
   (solder_mask_margin 0.102))
  (pad "CN10_34" thru_hole circle locked (at 31.75 31.13) (size 1.53 1.53) (drill 1.02) (layers "*.Cu" "*.Mask") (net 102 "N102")
   (solder_mask_margin 0.102))
  (pad "CN10_35" thru_hole circle locked (at 29.21 33.67) (size 1.53 1.53) (drill 1.02) (layers "*.Cu" "*.Mask") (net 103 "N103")
   (solder_mask_margin 0.102))
  (pad "CN10_36" thru_hole circle locked (at 31.75 33.67) (size 1.53 1.53) (drill 1.02) (layers "*.Cu" "*.Mask") (solder_mask_margin 0.102))
  (pad "CN10_37" thru_hole circle locked (at 29.21 36.21) (size 1.53 1.53) (drill 1.02) (layers "*.Cu" "*.Mask") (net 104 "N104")
   (solder_mask_margin 0.102))
  (pad "CN10_38" thru_hole circle locked (at 31.75 36.21) (size 1.53 1.53) (drill 1.02) (layers "*.Cu" "*.Mask") (solder_mask_margin 0.102)))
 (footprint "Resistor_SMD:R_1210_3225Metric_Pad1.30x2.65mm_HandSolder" (layer "F.Cu") (at 122.91 55.88)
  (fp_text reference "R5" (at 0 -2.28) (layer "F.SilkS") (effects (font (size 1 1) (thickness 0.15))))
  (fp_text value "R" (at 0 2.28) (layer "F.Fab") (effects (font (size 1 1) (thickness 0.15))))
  (pad "1" smd roundrect (at -1.55 0) (size 1.3 2.65) (layers "F.Cu" "F.Paste" "F.Mask") (roundrect_rratio 0.192308) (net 32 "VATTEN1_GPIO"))
  (pad "2" smd roundrect (at 1.55 0) (size 1.3 2.65) (layers "F.Cu" "F.Paste" "F.Mask") (roundrect_rratio 0.192308) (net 3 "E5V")))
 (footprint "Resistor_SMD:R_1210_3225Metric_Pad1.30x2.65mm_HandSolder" (layer "F.Cu") (at 84.55 76.2)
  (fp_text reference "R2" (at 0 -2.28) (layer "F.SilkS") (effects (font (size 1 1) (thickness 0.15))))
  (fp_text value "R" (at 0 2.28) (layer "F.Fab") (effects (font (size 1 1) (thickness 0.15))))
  (pad "1" smd roundrect (at -1.55 0) (size 1.3 2.65) (layers "F.Cu" "F.Paste" "F.Mask") (roundrect_rratio 0.192308) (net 33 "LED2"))
  (pad "2" smd roundrect (at 1.55 0) (size 1.3 2.65) (layers "F.Cu" "F.Paste" "F.Mask") (roundrect_rratio 0.192308) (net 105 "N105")))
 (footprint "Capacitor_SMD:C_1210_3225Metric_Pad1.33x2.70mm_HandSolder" (layer "F.Cu") (at 111.76 61.9375 90)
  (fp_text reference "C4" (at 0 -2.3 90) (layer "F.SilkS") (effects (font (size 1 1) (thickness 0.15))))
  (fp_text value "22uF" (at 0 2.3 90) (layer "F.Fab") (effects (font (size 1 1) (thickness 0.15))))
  (pad "1" smd roundrect (at -1.5625 0 90) (size 1.325 2.7) (layers "F.Cu" "F.Paste" "F.Mask") (roundrect_rratio 0.188679) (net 3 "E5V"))
  (pad "2" smd roundrect (at 1.5625 0 90) (size 1.325 2.7) (layers "F.Cu" "F.Paste" "F.Mask") (roundrect_rratio 0.188679) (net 5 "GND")))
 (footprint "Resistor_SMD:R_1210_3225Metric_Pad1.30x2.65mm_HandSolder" (layer "F.Cu") (at 84.55 83.82)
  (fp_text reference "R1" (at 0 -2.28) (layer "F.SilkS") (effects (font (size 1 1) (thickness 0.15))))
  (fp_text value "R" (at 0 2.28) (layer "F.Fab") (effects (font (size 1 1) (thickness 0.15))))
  (pad "1" smd roundrect (at -1.55 0) (size 1.3 2.65) (layers "F.Cu" "F.Paste" "F.Mask") (roundrect_rratio 0.192308) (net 31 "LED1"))
  (pad "2" smd roundrect (at 1.55 0) (size 1.3 2.65) (layers "F.Cu" "F.Paste" "F.Mask") (roundrect_rratio 0.192308) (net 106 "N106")))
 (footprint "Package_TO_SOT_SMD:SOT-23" (layer "F.Cu") (at 115.9025 55.88)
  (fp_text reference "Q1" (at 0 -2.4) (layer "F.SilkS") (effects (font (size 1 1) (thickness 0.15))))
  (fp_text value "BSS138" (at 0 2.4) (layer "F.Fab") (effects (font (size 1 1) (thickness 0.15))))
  (pad "1" smd roundrect (at -0.9375 -0.95) (size 1.475 0.6) (layers "F.Cu" "F.Paste" "F.Mask") (roundrect_rratio 0.25) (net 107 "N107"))
  (pad "2" smd roundrect (at -0.9375 0.95) (size 1.475 0.6) (layers "F.Cu" "F.Paste" "F.Mask") (roundrect_rratio 0.25) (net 5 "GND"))
  (pad "3" smd roundrect (at 0.9375 0) (size 1.475 0.6) (layers "F.Cu" "F.Paste" "F.Mask") (roundrect_rratio 0.25) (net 32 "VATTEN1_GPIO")))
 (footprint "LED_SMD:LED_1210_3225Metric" (layer "F.Cu") (at 92.84 76.2 180)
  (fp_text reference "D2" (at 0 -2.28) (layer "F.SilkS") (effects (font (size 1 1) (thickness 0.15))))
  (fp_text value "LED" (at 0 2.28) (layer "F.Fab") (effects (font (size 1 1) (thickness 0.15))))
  (pad "1" smd roundrect (at -1.4 0 180) (size 1.25 2.65) (layers "F.Cu" "F.Paste" "F.Mask") (roundrect_rratio 0.2) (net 5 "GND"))
  (pad "2" smd roundrect (at 1.4 0 180) (size 1.25 2.65) (layers "F.Cu" "F.Paste" "F.Mask") (roundrect_rratio 0.2) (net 105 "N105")))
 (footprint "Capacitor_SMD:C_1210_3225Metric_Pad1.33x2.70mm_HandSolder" (layer "F.Cu") (at 93.98 57.4425 -90)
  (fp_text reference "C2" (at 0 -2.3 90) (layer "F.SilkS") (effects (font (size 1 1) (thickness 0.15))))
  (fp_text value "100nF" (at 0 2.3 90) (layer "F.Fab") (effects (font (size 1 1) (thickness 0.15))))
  (pad "1" smd roundrect (at -1.5625 0 270) (size 1.325 2.7) (layers "F.Cu" "F.Paste" "F.Mask") (roundrect_rratio 0.188679) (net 6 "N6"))
  (pad "2" smd roundrect (at 1.5625 0 270) (size 1.325 2.7) (layers "F.Cu" "F.Paste" "F.Mask") (roundrect_rratio 0.188679) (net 7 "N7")))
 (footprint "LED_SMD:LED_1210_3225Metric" (layer "F.Cu") (at 92.84 68.58 180)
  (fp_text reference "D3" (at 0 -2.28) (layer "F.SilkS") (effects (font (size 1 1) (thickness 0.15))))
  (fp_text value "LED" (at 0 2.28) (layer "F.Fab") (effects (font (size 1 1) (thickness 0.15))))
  (pad "1" smd roundrect (at -1.4 0 180) (size 1.25 2.65) (layers "F.Cu" "F.Paste" "F.Mask") (roundrect_rratio 0.2) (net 5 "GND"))
  (pad "2" smd roundrect (at 1.4 0 180) (size 1.25 2.65) (layers "F.Cu" "F.Paste" "F.Mask") (roundrect_rratio 0.2) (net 2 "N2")))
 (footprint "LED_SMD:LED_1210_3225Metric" (layer "F.Cu") (at 92.84 83.82 180)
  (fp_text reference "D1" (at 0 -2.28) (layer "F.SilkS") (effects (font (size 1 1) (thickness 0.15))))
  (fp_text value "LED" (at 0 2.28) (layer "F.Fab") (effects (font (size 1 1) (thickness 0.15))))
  (pad "1" smd roundrect (at -1.4 0 180) (size 1.25 2.65) (layers "F.Cu" "F.Paste" "F.Mask") (roundrect_rratio 0.2) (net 5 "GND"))
  (pad "2" smd roundrect (at 1.4 0 180) (size 1.25 2.65) (layers "F.Cu" "F.Paste" "F.Mask") (roundrect_rratio 0.2) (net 106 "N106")))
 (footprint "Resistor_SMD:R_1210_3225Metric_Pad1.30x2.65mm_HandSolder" (layer "F.Cu") (at 108.23 53.34)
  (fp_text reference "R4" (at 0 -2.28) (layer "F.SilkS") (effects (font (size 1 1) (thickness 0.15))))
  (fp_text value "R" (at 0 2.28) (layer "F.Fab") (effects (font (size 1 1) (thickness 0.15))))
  (pad "1" smd roundrect (at -1.55 0) (size 1.3 2.65) (layers "F.Cu" "F.Paste" "F.Mask") (roundrect_rratio 0.192308)
   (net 8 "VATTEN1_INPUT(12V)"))
  (pad "2" smd roundrect (at 1.55 0) (size 1.3 2.65) (layers "F.Cu" "F.Paste" "F.Mask") (roundrect_rratio 0.192308) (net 107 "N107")))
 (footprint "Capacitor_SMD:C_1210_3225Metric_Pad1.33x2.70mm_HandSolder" (layer "F.Cu") (at 100.6225 50.8 180)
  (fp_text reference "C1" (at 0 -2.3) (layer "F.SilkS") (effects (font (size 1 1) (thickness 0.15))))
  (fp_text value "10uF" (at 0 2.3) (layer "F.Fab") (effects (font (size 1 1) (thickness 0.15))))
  (pad "1" smd roundrect (at -1.5625 0 180) (size 1.325 2.7) (layers "F.Cu" "F.Paste" "F.Mask") (roundrect_rratio 0.188679) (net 4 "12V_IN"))
  (pad "2" smd roundrect (at 1.5625 0 180) (size 1.325 2.7) (layers "F.Cu" "F.Paste" "F.Mask") (roundrect_rratio 0.188679) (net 5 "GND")))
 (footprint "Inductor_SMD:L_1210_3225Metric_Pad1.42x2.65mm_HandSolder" (layer "F.Cu") (at 100.5475 66.04)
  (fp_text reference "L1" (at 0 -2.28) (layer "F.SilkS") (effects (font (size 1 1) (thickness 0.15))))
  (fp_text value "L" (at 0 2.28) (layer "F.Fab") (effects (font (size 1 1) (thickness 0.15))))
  (pad "1" smd roundrect (at -1.4875 0) (size 1.425 2.65) (layers "F.Cu" "F.Paste" "F.Mask") (roundrect_rratio 0.175439) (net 6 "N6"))
  (pad "2" smd roundrect (at 1.4875 0) (size 1.425 2.65) (layers "F.Cu" "F.Paste" "F.Mask") (roundrect_rratio 0.175439) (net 3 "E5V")))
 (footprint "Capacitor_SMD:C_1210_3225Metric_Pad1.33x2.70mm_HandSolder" (layer "F.Cu") (at 106.68 61.9375 90)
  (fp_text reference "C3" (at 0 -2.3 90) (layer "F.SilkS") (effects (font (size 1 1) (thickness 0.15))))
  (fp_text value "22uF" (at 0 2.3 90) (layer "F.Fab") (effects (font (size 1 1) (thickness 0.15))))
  (pad "1" smd roundrect (at -1.5625 0 90) (size 1.325 2.7) (layers "F.Cu" "F.Paste" "F.Mask") (roundrect_rratio 0.188679) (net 3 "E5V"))
  (pad "2" smd roundrect (at 1.5625 0 90) (size 1.325 2.7) (layers "F.Cu" "F.Paste" "F.Mask") (roundrect_rratio 0.188679) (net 5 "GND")))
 (gr_rect locked (start 63.03 43.98) (end 163.03 143.98) (stroke (width 0.1) (type default)) (fill none) (layer "Edge.Cuts"))
 (segment (start 94.24 68.58) (end 94.24 66.3) (width 0.25) (layer "F.Cu") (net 5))
 (segment (start 99.06 50.8) (end 99.06 56.52) (width 0.25) (layer "F.Cu") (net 5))
 (segment (start 104.14 57.835) (end 104.14 53.34) (width 0.25) (layer "F.Cu") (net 5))
 (segment (start 94.24 83.82) (end 94.24 76.2) (width 0.25) (layer "F.Cu") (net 5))
 (segment (start 99.06 50.8) (end 99.06 45.72) (width 0.25) (layer "F.Cu") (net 5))
 (segment (start 106.68 60.375) (end 111.76 60.375) (width 0.25) (layer "F.Cu") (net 5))
 (segment (start 111.76 60.375) (end 111.76 60.035) (width 0.25) (layer "F.Cu") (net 5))
 (segment (start 88.9 60.96) (end 88.9 55.88) (width 0.25) (layer "F.Cu") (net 5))
 (segment (start 93.98 50.8) (end 99.06 50.8) (width 0.25) (layer "F.Cu") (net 5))
 (segment (start 88.9 55.88) (end 93.98 50.8) (width 0.25) (layer "F.Cu") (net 5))
 (segment (start 94.24 66.3) (end 88.9 60.96) (width 0.25) (layer "F.Cu") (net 5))
 (segment (start 106.68 60.375) (end 104.14 57.835) (width 0.25) (layer "F.Cu") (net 5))
 (segment (start 111.76 60.035) (end 114.965 56.83) (width 0.25) (layer "F.Cu") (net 5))
 (segment (start 94.24 76.2) (end 94.24 68.58) (width 0.25) (layer "F.Cu") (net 5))
 (via (at 104.14 53.34) (size 0.8) (drill 0.4) (layers "F.Cu" "B.Cu") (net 5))
 (segment (start 99.06 48.26) (end 99.06 45.72) (width 0.25) (layer "B.Cu") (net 5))
 (segment (start 83.82 114.95) (end 81.28 114.95) (width 0.25) (layer "B.Cu") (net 5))
 (segment (start 147.32 88.9) (end 139.7 88.9) (width 0.25) (layer "B.Cu") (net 5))
 (segment (start 88.9 114.95) (end 86.36 112.41) (width 0.25) (layer "B.Cu") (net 5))
 (segment (start 83.82 99.71) (end 86.36 102.25) (width 0.25) (layer "B.Cu") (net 5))
 (segment (start 146.67 114.95) (end 147.32 114.3) (width 0.25) (layer "B.Cu") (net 5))
 (segment (start 144.78 114.95) (end 146.67 114.95) (width 0.25) (layer "B.Cu") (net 5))
 (segment (start 104.14 53.34) (end 104.14 86.36) (width 0.25) (layer "B.Cu") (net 5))
 (segment (start 91.44 99.06) (end 88.9 99.06) (width 0.25) (layer "B.Cu") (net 5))
 (segment (start 83.82 117.49) (end 83.82 114.95) (width 0.25) (layer "B.Cu") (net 5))
 (segment (start 104.14 53.34) (end 139.7 88.9) (width 0.25) (layer "B.Cu") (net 5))
 (segment (start 88.9 117.49) (end 88.9 114.95) (width 0.25) (layer "B.Cu") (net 5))
 (segment (start 88.25 99.71) (end 83.82 99.71) (width 0.25) (layer "B.Cu") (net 5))
 (segment (start 104.14 86.36) (end 91.44 99.06) (width 0.25) (layer "B.Cu") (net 5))
 (segment (start 86.36 102.25) (end 86.36 112.41) (width 0.25) (layer "B.Cu") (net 5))
 (segment (start 147.32 114.3) (end 147.32 88.9) (width 0.25) (layer "B.Cu") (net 5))
 (segment (start 88.9 99.06) (end 88.25 99.71) (width 0.25) (layer "B.Cu") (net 5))
 (segment (start 139.7 99.71) (end 142.24 102.25) (width 0.25) (layer "B.Cu") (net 5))
 (segment (start 86.36 112.41) (end 83.82 114.95) (width 0.25) (layer "B.Cu") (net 5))
 (segment (start 104.14 53.34) (end 99.06 48.26) (width 0.25) (layer "B.Cu") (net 5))
 (segment (start 147.32 127.65) (end 144.78 130.19) (width 0.25) (layer "B.Cu") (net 5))
 (segment (start 139.7 88.9) (end 139.7 99.71) (width 0.25) (layer "B.Cu") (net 5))
 (segment (start 147.32 114.3) (end 147.32 127.65) (width 0.25) (layer "B.Cu") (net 5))
 (segment (start 86.1 83.82) (end 91.44 83.82) (width 0.25) (layer "F.Cu") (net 106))
 (segment (start 86.1 76.2) (end 91.44 76.2) (width 0.25) (layer "F.Cu") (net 105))
 (segment (start 86.1 68.58) (end 91.44 68.58) (width 0.25) (layer "F.Cu") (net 2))
 (segment (start 113.375 53.34) (end 114.965 54.93) (width 0.25) (layer "F.Cu") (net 107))
 (segment (start 109.78 53.34) (end 113.375 53.34) (width 0.25) (layer "F.Cu") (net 107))
 (segment (start 83 83.82) (end 81.28 85.54) (width 0.25) (layer "F.Cu") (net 31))
 (segment (start 81.28 85.54) (end 81.28 92.09) (width 0.25) (layer "F.Cu") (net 31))
 (segment (start 83 76.2) (end 81.28 76.2) (width 0.25) (layer "F.Cu") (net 33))
 (segment (start 79.19 92.54) (end 81.28 94.63) (width 0.25) (layer "F.Cu") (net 33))
 (segment (start 81.28 76.2) (end 79.19 78.29) (width 0.25) (layer "F.Cu") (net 33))
 (segment (start 79.19 78.29) (end 79.19 92.54) (width 0.25) (layer "F.Cu") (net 33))
 (segment (start 78.74 71.12) (end 78.74 106.68) (width 0.25) (layer "F.Cu") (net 1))
 (segment (start 83 68.58) (end 81.28 68.58) (width 0.25) (layer "F.Cu") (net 1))
 (segment (start 78.74 106.68) (end 79.39 107.33) (width 0.25) (layer "F.Cu") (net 1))
 (segment (start 81.28 68.58) (end 78.74 71.12) (width 0.25) (layer "F.Cu") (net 1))
 (segment (start 79.39 107.33) (end 81.28 107.33) (width 0.25) (layer "F.Cu") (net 1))
 (segment (start 104.14 83.82) (end 101.6 86.36) (width 0.25) (layer "F.Cu") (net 32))
 (segment (start 116.84 71.12) (end 104.14 83.82) (width 0.25) (layer "F.Cu") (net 32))
 (segment (start 116.84 55.88) (end 116.84 71.12) (width 0.25) (layer "F.Cu") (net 32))
 (segment (start 116.84 55.88) (end 121.36 55.88) (width 0.25) (layer "F.Cu") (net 32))
 (via (at 101.6 86.36) (size 0.8) (drill 0.4) (layers "F.Cu" "B.Cu") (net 32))
 (segment (start 93.98 86.36) (end 88.25 92.09) (width 0.25) (layer "B.Cu") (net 32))
 (segment (start 88.25 92.09) (end 83.82 92.09) (width 0.25) (layer "B.Cu") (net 32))
 (segment (start 101.6 86.36) (end 93.98 86.36) (width 0.25) (layer "B.Cu") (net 32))
 (segment (start 102.185 50.8) (end 101.335 51.65) (width 0.25) (layer "F.Cu") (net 4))
 (segment (start 101.6 50.215) (end 101.6 45.72) (width 0.25) (layer "F.Cu") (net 4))
 (segment (start 102.185 50.8) (end 101.6 50.215) (width 0.25) (layer "F.Cu") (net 4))
 (segment (start 101.335 56.52) (end 101.335 57.47) (width 0.25) (layer "F.Cu") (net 4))
 (segment (start 101.335 51.65) (end 101.335 56.52) (width 0.25) (layer "F.Cu") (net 4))
 (segment (start 91.44 60.96) (end 91.44 58.42) (width 0.25) (layer "F.Cu") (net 6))
 (segment (start 95.57 57.47) (end 99.06 57.47) (width 0.25) (layer "F.Cu") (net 6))
 (segment (start 96.52 63.5) (end 93.98 63.5) (width 0.25) (layer "F.Cu") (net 6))
 (segment (start 99.06 66.04) (end 96.52 63.5) (width 0.25) (layer "F.Cu") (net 6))
 (segment (start 91.44 58.42) (end 93.98 55.88) (width 0.25) (layer "F.Cu") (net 6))
 (segment (start 93.98 63.5) (end 91.44 60.96) (width 0.25) (layer "F.Cu") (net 6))
 (segment (start 93.98 55.88) (end 95.57 57.47) (width 0.25) (layer "F.Cu") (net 6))
 (segment (start 94.565 58.42) (end 99.06 58.42) (width 0.25) (layer "F.Cu") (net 7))
 (segment (start 93.98 59.005) (end 94.565 58.42) (width 0.25) (layer "F.Cu") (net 7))
 (segment (start 102.035 83.385) (end 88.25 97.17) (width 0.25) (layer "F.Cu") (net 3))
 (segment (start 106.68 63.5) (end 111.76 63.5) (width 0.25) (layer "F.Cu") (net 3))
 (segment (start 102.035 66.04) (end 104.14 66.04) (width 0.25) (layer "F.Cu") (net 3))
 (segment (start 114.3 60.96) (end 111.76 63.5) (width 0.25) (layer "F.Cu") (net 3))
 (segment (start 102.035 66.04) (end 102.035 83.385) (width 0.25) (layer "F.Cu") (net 3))
 (segment (start 124.46 55.88) (end 119.38 60.96) (width 0.25) (layer "F.Cu") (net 3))
 (segment (start 106.68 63.5) (end 101.6 58.42) (width 0.25) (layer "F.Cu") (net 3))
 (segment (start 88.25 97.17) (end 83.82 97.17) (width 0.25) (layer "F.Cu") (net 3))
 (segment (start 101.6 58.42) (end 101.335 58.42) (width 0.25) (layer "F.Cu") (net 3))
 (segment (start 104.14 66.04) (end 106.68 63.5) (width 0.25) (layer "F.Cu") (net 3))
 (segment (start 119.38 60.96) (end 119.38 63.5) (width 0.25) (layer "F.Cu") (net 3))
 (via (at 119.38 63.5) (size 0.8) (drill 0.4) (layers "F.Cu" "B.Cu") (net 3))
 (via (at 114.3 60.96) (size 0.8) (drill 0.4) (layers "F.Cu" "B.Cu") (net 3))
 (segment (start 116.84 63.5) (end 114.3 60.96) (width 0.25) (layer "B.Cu") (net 3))
 (segment (start 119.38 63.5) (end 116.84 63.5) (width 0.25) (layer "B.Cu") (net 3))
 (segment (start 104.14 50.8) (end 104.14 45.72) (width 0.25) (layer "F.Cu") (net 8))
 (segment (start 106.68 53.34) (end 104.14 50.8) (width 0.25) (layer "F.Cu") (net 8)))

